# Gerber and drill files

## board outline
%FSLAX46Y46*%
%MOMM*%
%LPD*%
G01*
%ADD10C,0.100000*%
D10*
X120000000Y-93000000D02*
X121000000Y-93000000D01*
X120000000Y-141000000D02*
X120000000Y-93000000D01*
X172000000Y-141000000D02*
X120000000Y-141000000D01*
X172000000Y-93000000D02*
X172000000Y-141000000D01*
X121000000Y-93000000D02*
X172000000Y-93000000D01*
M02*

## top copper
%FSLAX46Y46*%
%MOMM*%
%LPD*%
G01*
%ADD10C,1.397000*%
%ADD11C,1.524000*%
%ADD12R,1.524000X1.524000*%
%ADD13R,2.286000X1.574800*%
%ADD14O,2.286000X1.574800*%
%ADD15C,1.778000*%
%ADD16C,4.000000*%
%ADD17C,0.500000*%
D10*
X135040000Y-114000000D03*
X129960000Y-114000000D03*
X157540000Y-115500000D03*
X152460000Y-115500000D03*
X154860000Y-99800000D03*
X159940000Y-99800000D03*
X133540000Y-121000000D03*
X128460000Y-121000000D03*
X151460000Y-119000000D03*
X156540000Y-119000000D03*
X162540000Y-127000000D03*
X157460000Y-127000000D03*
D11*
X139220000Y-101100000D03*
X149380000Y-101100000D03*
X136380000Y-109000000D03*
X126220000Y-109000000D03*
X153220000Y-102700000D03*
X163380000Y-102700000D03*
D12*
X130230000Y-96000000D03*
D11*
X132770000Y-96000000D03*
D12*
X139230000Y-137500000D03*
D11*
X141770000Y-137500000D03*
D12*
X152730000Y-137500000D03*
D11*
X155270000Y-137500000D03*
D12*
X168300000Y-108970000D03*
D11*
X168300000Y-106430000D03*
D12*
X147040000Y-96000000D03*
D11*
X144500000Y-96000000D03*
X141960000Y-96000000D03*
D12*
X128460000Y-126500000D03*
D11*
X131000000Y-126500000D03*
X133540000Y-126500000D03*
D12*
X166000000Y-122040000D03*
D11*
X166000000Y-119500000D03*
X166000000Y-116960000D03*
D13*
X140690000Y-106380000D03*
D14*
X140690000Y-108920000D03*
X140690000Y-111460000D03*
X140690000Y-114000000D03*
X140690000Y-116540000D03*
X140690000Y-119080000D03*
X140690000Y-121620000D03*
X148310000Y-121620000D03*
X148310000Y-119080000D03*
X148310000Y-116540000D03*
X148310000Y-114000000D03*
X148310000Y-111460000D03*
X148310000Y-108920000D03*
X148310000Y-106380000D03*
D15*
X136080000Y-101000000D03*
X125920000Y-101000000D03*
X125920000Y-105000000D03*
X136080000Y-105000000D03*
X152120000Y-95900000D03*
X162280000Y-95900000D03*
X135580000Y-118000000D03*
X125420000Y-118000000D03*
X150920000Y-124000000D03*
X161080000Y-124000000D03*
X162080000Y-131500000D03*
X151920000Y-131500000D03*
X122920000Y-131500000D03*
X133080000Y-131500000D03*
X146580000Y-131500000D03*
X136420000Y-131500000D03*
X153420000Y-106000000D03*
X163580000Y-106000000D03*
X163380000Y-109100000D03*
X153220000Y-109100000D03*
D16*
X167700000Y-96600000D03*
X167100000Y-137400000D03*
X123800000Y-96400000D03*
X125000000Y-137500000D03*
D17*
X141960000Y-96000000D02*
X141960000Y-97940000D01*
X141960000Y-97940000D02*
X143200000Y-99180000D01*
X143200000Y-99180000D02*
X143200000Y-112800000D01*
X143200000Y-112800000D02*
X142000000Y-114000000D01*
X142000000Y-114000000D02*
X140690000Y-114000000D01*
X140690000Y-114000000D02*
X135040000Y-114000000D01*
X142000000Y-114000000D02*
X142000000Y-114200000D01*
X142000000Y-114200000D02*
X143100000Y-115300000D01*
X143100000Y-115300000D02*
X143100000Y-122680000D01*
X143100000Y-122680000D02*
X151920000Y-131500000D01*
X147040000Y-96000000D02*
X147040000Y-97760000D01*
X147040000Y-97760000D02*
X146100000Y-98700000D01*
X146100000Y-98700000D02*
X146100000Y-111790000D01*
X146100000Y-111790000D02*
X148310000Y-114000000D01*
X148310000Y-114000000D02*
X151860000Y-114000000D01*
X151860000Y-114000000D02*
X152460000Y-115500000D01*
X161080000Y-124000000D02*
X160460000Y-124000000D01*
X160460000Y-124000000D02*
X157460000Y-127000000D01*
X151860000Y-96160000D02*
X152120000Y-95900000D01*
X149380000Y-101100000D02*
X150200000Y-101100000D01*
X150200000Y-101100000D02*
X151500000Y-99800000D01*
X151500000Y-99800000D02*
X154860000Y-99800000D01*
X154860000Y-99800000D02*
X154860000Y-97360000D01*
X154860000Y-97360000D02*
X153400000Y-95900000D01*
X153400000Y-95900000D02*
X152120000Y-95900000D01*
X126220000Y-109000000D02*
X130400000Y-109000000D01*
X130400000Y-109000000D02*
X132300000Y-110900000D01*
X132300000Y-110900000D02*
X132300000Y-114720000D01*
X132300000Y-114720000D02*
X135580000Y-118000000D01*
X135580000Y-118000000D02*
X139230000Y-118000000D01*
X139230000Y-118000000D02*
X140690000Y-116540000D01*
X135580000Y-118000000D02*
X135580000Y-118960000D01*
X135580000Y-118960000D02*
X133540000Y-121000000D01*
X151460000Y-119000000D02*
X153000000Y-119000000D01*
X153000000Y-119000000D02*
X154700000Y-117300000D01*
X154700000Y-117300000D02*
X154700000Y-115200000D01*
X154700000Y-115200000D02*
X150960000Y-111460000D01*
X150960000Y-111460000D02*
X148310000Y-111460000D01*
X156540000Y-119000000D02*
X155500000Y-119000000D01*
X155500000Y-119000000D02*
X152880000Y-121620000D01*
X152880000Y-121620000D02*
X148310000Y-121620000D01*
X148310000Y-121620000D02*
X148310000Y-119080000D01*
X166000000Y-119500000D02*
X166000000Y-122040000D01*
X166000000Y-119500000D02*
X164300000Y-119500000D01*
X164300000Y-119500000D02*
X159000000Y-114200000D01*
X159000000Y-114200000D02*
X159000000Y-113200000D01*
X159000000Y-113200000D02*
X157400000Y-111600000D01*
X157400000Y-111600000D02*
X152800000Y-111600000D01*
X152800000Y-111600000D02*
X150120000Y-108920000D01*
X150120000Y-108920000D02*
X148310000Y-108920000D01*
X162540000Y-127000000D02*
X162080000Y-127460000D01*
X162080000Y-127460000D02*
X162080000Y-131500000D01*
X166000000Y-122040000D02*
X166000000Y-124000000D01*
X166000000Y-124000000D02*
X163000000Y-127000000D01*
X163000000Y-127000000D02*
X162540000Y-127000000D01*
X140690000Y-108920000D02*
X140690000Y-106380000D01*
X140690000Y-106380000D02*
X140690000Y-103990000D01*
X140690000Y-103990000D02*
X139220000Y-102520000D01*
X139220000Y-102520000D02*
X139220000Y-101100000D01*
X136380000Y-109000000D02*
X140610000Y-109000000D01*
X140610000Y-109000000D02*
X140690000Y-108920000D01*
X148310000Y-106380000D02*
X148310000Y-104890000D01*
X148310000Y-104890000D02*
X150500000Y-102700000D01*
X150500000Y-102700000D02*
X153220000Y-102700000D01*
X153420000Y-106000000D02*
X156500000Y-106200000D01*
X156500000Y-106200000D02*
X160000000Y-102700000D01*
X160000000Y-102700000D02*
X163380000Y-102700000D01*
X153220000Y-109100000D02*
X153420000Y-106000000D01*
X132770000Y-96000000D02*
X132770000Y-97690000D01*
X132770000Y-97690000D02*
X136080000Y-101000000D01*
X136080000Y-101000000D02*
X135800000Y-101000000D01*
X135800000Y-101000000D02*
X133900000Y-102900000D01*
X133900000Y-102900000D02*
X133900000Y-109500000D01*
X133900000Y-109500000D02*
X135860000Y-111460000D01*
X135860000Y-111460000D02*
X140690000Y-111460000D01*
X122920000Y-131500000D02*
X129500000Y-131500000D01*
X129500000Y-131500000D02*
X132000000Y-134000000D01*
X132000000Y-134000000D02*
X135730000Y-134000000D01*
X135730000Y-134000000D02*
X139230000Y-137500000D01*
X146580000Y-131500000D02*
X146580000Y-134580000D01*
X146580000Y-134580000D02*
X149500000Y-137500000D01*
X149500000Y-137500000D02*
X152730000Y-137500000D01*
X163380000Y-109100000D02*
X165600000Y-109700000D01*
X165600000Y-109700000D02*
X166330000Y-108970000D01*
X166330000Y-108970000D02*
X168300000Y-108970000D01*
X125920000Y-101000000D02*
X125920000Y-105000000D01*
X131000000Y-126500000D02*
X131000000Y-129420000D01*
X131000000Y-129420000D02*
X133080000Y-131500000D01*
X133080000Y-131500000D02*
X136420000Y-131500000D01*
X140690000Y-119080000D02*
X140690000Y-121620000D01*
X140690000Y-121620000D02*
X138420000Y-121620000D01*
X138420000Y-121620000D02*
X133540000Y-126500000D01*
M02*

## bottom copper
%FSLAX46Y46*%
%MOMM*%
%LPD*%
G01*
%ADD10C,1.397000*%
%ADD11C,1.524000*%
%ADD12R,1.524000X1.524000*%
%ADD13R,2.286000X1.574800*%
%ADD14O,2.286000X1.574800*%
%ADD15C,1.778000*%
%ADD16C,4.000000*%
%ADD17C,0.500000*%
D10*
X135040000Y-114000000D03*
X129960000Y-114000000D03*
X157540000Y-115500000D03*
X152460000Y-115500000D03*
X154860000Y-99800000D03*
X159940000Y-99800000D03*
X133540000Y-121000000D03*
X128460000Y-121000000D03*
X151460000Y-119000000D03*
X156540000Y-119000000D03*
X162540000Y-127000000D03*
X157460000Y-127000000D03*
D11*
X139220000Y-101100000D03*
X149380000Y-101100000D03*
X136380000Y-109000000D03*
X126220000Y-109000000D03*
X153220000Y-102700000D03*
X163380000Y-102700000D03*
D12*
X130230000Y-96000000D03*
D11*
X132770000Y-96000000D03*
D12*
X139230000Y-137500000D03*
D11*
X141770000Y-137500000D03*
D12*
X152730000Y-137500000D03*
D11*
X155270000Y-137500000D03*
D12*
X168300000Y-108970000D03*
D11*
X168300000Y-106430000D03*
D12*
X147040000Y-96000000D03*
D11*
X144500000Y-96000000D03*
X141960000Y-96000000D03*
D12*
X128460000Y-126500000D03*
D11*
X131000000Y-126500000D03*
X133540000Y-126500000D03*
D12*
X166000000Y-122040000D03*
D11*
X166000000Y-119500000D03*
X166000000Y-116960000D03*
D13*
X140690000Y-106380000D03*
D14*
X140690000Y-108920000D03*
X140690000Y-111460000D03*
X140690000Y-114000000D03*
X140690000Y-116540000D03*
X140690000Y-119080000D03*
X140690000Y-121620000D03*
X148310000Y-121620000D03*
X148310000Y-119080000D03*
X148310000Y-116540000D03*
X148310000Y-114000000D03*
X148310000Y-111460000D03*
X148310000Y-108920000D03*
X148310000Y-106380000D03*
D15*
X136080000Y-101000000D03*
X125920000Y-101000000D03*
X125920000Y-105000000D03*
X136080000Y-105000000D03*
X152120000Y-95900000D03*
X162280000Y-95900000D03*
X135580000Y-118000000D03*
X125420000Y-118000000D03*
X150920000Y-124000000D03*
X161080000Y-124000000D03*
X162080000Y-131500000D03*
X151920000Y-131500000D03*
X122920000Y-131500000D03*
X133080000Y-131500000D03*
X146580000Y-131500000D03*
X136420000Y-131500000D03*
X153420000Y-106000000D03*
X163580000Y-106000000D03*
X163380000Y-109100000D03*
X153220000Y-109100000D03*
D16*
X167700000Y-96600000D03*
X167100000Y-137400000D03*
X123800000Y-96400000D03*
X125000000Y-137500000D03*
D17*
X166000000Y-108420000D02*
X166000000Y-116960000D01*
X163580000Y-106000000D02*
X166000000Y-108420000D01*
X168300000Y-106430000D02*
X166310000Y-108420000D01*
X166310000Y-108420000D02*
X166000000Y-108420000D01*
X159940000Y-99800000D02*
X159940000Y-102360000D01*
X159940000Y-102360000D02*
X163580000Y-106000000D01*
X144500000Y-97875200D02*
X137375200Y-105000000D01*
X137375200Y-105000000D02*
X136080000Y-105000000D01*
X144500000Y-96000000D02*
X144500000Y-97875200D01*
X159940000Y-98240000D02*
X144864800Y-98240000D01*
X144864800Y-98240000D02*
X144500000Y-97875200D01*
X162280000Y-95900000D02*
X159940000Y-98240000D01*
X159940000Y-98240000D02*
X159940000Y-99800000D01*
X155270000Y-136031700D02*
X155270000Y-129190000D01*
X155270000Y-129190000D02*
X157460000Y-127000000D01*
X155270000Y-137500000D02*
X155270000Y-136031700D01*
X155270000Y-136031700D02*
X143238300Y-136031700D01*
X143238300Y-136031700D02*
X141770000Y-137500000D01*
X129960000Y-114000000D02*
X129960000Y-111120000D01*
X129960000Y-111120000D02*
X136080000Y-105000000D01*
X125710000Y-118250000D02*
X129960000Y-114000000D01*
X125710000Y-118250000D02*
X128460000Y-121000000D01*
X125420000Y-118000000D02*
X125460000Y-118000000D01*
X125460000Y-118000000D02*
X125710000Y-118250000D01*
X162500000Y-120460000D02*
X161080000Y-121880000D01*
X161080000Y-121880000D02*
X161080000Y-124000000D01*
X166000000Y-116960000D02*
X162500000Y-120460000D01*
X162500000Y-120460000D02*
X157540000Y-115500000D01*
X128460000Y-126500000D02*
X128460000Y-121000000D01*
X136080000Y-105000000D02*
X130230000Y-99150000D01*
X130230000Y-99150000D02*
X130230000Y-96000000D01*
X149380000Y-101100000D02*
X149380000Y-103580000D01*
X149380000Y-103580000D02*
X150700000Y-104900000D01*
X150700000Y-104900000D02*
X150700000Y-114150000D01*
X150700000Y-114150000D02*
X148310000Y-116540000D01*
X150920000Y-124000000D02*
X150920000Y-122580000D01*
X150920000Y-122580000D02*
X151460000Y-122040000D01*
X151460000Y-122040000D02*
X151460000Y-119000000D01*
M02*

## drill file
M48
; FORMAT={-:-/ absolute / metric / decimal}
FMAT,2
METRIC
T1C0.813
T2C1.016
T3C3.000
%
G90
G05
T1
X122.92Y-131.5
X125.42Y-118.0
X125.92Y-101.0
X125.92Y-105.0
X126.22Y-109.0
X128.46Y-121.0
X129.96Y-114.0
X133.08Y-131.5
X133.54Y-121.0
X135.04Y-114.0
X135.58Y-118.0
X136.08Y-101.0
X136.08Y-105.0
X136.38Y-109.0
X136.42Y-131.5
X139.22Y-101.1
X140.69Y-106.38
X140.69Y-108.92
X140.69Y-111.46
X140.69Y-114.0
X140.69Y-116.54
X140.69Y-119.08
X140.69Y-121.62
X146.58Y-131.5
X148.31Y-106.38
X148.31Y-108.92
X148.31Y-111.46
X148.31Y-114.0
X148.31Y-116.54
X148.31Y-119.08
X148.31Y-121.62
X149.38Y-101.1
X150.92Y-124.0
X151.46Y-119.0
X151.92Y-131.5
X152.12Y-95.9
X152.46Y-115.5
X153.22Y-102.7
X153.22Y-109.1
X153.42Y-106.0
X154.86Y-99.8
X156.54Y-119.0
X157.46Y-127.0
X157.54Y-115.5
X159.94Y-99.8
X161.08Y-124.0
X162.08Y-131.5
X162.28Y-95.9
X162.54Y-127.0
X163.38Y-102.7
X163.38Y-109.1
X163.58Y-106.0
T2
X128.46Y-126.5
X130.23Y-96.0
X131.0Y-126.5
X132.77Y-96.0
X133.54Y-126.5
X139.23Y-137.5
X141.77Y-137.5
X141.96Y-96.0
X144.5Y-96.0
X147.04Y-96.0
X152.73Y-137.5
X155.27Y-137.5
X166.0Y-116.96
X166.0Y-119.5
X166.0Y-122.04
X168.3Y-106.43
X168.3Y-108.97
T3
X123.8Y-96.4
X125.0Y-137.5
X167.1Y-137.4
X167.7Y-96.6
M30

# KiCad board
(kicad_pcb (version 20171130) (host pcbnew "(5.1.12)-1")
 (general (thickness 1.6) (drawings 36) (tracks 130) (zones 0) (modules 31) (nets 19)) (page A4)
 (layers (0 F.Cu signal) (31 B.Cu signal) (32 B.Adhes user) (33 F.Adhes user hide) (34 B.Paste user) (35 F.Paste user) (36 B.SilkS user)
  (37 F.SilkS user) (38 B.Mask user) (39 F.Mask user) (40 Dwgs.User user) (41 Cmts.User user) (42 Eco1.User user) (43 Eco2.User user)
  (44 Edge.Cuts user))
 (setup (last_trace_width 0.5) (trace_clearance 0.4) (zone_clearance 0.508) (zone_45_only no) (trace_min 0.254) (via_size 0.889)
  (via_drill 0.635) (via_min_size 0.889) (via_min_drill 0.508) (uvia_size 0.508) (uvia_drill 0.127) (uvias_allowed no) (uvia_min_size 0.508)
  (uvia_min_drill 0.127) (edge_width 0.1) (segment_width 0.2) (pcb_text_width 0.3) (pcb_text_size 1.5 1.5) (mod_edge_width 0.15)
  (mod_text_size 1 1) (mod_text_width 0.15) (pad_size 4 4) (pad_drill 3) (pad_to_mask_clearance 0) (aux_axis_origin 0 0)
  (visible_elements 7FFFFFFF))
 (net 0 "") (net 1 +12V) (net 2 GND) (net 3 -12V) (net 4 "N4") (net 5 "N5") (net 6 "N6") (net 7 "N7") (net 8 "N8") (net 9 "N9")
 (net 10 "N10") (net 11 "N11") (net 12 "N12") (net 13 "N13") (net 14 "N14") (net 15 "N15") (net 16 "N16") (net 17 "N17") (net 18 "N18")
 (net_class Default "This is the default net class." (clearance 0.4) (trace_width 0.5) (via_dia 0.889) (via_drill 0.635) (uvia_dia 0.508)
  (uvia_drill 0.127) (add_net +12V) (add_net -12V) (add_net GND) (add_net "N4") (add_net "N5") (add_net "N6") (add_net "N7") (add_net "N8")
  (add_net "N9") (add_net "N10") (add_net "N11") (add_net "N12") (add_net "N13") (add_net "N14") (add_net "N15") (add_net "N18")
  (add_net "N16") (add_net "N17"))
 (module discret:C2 (layer F.Cu) (at 132.5 114 180)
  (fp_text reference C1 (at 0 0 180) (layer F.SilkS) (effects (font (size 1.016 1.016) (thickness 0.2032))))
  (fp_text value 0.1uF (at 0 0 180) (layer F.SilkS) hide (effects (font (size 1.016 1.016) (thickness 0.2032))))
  (pad 1 thru_hole circle (at -2.54 0 180) (size 1.397 1.397) (drill 0.8128) (layers *.Cu *.Mask F.SilkS) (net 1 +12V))
  (pad 2 thru_hole circle (at 2.54 0 180) (size 1.397 1.397) (drill 0.8128) (layers *.Cu *.Mask F.SilkS) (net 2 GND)))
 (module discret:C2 (layer F.Cu) (at 155 115.5 180)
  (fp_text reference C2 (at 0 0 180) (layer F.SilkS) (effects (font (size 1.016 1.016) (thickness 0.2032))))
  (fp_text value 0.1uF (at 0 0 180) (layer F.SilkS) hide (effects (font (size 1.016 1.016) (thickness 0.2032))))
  (pad 1 thru_hole circle (at -2.54 0 180) (size 1.397 1.397) (drill 0.8128) (layers *.Cu *.Mask F.SilkS) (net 2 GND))
  (pad 2 thru_hole circle (at 2.54 0 180) (size 1.397 1.397) (drill 0.8128) (layers *.Cu *.Mask F.SilkS) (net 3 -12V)))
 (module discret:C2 (layer F.Cu) (at 157.4 99.8)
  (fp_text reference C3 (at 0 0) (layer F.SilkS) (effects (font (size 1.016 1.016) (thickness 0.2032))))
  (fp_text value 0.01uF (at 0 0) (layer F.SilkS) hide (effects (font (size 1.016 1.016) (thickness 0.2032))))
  (pad 1 thru_hole circle (at -2.54 0) (size 1.397 1.397) (drill 0.8128) (layers *.Cu *.Mask F.SilkS) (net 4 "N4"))
  (pad 2 thru_hole circle (at 2.54 0) (size 1.397 1.397) (drill 0.8128) (layers *.Cu *.Mask F.SilkS) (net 2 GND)))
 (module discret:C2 (layer F.Cu) (at 131 121 180)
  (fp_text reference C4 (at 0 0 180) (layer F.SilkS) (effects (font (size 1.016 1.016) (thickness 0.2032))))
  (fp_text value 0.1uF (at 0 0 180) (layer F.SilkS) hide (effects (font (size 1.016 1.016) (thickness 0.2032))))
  (pad 1 thru_hole circle (at -2.54 0 180) (size 1.397 1.397) (drill 0.8128) (layers *.Cu *.Mask F.SilkS) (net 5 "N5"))
  (pad 2 thru_hole circle (at 2.54 0 180) (size 1.397 1.397) (drill 0.8128) (layers *.Cu *.Mask F.SilkS) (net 2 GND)))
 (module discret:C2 (layer F.Cu) (at 154 119)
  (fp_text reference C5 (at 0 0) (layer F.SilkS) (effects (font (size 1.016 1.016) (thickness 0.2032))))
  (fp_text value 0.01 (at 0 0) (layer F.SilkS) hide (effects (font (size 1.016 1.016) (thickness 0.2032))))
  (pad 1 thru_hole circle (at -2.54 0) (size 1.397 1.397) (drill 0.8128) (layers *.Cu *.Mask F.SilkS) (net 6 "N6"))
  (pad 2 thru_hole circle (at 2.54 0) (size 1.397 1.397) (drill 0.8128) (layers *.Cu *.Mask F.SilkS) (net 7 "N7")))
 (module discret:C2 (layer F.Cu) (at 160 127 180)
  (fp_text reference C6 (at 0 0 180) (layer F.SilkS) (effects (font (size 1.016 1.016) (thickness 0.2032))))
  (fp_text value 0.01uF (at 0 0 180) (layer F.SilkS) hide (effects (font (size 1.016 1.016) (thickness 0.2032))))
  (pad 1 thru_hole circle (at -2.54 0 180) (size 1.397 1.397) (drill 0.8128) (layers *.Cu *.Mask F.SilkS) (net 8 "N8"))
  (pad 2 thru_hole circle (at 2.54 0 180) (size 1.397 1.397) (drill 0.8128) (layers *.Cu *.Mask F.SilkS) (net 2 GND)))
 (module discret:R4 (layer F.Cu) (at 144.3 101.1) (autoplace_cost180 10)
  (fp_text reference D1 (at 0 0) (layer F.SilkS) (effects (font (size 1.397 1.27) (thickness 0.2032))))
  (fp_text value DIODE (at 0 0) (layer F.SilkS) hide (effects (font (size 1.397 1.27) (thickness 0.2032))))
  (pad 1 thru_hole circle (at -5.08 0) (size 1.524 1.524) (drill 0.8128) (layers *.Cu *.Mask F.SilkS) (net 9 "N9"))
  (pad 2 thru_hole circle (at 5.08 0) (size 1.524 1.524) (drill 0.8128) (layers *.Cu *.Mask F.SilkS) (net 4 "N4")))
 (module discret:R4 (layer F.Cu) (at 131.3 109 180) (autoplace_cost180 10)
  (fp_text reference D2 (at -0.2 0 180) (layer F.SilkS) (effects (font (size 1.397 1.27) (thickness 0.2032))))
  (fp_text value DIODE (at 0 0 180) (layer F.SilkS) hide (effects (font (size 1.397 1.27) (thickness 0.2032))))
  (pad 1 thru_hole circle (at -5.08 0 180) (size 1.524 1.524) (drill 0.8128) (layers *.Cu *.Mask F.SilkS) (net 9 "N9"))
  (pad 2 thru_hole circle (at 5.08 0 180) (size 1.524 1.524) (drill 0.8128) (layers *.Cu *.Mask F.SilkS) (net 5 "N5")))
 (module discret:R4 (layer F.Cu) (at 158.3 102.7) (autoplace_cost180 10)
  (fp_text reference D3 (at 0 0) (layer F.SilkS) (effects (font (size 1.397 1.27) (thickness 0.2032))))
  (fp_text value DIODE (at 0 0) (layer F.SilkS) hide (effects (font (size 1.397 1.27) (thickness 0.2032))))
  (pad 1 thru_hole circle (at -5.08 0) (size 1.524 1.524) (drill 0.8128) (layers *.Cu *.Mask F.SilkS) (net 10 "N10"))
  (pad 2 thru_hole circle (at 5.08 0) (size 1.524 1.524) (drill 0.8128) (layers *.Cu *.Mask F.SilkS) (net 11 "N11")))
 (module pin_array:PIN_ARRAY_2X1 (layer F.Cu) (at 131.5 96)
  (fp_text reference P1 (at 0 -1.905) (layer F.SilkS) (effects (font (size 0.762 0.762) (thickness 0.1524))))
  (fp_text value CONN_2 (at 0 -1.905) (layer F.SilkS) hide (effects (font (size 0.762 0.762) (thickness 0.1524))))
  (pad 1 thru_hole rect (at -1.27 0) (size 1.524 1.524) (drill 1.016) (layers *.Cu *.Mask F.SilkS) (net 2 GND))
  (pad 2 thru_hole circle (at 1.27 0) (size 1.524 1.524) (drill 1.016) (layers *.Cu *.Mask F.SilkS) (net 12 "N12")))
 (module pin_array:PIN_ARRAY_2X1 (layer F.Cu) (at 140.5 137.5)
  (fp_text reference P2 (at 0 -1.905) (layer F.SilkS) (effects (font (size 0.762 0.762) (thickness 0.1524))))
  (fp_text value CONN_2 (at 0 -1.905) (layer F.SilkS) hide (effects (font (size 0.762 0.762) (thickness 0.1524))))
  (pad 1 thru_hole rect (at -1.27 0) (size 1.524 1.524) (drill 1.016) (layers *.Cu *.Mask F.SilkS) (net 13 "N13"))
  (pad 2 thru_hole circle (at 1.27 0) (size 1.524 1.524) (drill 1.016) (layers *.Cu *.Mask F.SilkS) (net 2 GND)))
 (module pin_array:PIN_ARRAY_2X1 (layer F.Cu) (at 154 137.5)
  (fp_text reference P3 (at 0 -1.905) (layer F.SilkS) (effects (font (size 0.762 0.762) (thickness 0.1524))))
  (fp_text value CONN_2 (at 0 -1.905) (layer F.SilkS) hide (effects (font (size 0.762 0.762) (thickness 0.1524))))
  (pad 1 thru_hole rect (at -1.27 0) (size 1.524 1.524) (drill 1.016) (layers *.Cu *.Mask F.SilkS) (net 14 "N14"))
  (pad 2 thru_hole circle (at 1.27 0) (size 1.524 1.524) (drill 1.016) (layers *.Cu *.Mask F.SilkS) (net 2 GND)))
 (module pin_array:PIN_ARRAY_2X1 (layer F.Cu) (at 168.3 107.7 90)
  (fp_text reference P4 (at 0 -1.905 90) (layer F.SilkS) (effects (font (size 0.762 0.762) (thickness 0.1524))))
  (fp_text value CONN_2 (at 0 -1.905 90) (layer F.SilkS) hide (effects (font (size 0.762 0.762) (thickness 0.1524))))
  (pad 1 thru_hole rect (at -1.27 0 90) (size 1.524 1.524) (drill 1.016) (layers *.Cu *.Mask F.SilkS) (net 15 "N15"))
  (pad 2 thru_hole circle (at 1.27 0 90) (size 1.524 1.524) (drill 1.016) (layers *.Cu *.Mask F.SilkS) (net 2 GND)))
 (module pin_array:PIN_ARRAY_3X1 (layer F.Cu) (at 144.5 96 180)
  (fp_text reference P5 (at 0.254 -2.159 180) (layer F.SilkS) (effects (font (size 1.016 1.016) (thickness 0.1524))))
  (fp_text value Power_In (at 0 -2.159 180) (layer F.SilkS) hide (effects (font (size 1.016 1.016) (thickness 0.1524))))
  (pad 1 thru_hole rect (at -2.54 0 180) (size 1.524 1.524) (drill 1.016) (layers *.Cu *.Mask F.SilkS) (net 3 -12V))
  (pad 2 thru_hole circle (at 0 0 180) (size 1.524 1.524) (drill 1.016) (layers *.Cu *.Mask F.SilkS) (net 2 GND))
  (pad 3 thru_hole circle (at 2.54 0 180) (size 1.524 1.524) (drill 1.016) (layers *.Cu *.Mask F.SilkS) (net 1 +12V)))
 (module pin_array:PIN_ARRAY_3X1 (layer F.Cu) (at 131 126.5)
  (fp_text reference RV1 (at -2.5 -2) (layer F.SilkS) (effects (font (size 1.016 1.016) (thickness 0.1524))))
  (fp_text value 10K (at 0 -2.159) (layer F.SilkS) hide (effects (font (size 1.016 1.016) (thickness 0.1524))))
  (pad 1 thru_hole rect (at -2.54 0) (size 1.524 1.524) (drill 1.016) (layers *.Cu *.Mask F.SilkS) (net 2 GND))
  (pad 2 thru_hole circle (at 0 0) (size 1.524 1.524) (drill 1.016) (layers *.Cu *.Mask F.SilkS) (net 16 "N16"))
  (pad 3 thru_hole circle (at 2.54 0) (size 1.524 1.524) (drill 1.016) (layers *.Cu *.Mask F.SilkS) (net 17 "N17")))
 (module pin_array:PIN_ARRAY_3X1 (layer F.Cu) (at 166 119.5 90)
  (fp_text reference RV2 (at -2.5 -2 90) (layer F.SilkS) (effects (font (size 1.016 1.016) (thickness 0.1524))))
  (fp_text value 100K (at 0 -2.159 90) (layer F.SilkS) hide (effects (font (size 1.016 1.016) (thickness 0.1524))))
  (pad 1 thru_hole rect (at -2.54 0 90) (size 1.524 1.524) (drill 1.016) (layers *.Cu *.Mask F.SilkS) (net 8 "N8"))
  (pad 2 thru_hole circle (at 0 0 90) (size 1.524 1.524) (drill 1.016) (layers *.Cu *.Mask F.SilkS) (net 8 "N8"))
  (pad 3 thru_hole circle (at 2.54 0 90) (size 1.524 1.524) (drill 1.016) (layers *.Cu *.Mask F.SilkS) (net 2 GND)))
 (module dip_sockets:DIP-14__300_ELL (layer F.Cu) (at 144.5 114 270)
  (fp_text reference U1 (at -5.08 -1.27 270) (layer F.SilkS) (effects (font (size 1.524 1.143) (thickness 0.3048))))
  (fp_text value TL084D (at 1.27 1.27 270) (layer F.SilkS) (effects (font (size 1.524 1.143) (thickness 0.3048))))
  (pad 1 thru_hole rect (at -7.62 3.81 270) (size 1.5748 2.286) (drill 0.8128) (layers *.Cu *.Mask F.SilkS) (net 9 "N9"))
  (pad 2 thru_hole oval (at -5.08 3.81 270) (size 1.5748 2.286) (drill 0.8128) (layers *.Cu *.Mask F.SilkS) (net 9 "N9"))
  (pad 3 thru_hole oval (at -2.54 3.81 270) (size 1.5748 2.286) (drill 0.8128) (layers *.Cu *.Mask F.SilkS) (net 12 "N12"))
  (pad 4 thru_hole oval (at 0 3.81 270) (size 1.5748 2.286) (drill 0.8128) (layers *.Cu *.Mask F.SilkS) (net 1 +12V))
  (pad 5 thru_hole oval (at 2.54 3.81 270) (size 1.5748 2.286) (drill 0.8128) (layers *.Cu *.Mask F.SilkS) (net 5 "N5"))
  (pad 6 thru_hole oval (at 5.08 3.81 270) (size 1.5748 2.286) (drill 0.8128) (layers *.Cu *.Mask F.SilkS) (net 17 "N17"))
  (pad 7 thru_hole oval (at 7.62 3.81 270) (size 1.5748 2.286) (drill 0.8128) (layers *.Cu *.Mask F.SilkS) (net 17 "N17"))
  (pad 8 thru_hole oval (at 7.62 -3.81 270) (size 1.5748 2.286) (drill 0.8128) (layers *.Cu *.Mask F.SilkS) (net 7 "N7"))
  (pad 9 thru_hole oval (at 5.08 -3.81 270) (size 1.5748 2.286) (drill 0.8128) (layers *.Cu *.Mask F.SilkS) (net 7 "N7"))
  (pad 10 thru_hole oval (at 2.54 -3.81 270) (size 1.5748 2.286) (drill 0.8128) (layers *.Cu *.Mask F.SilkS) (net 4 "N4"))
  (pad 11 thru_hole oval (at 0 -3.81 270) (size 1.5748 2.286) (drill 0.8128) (layers *.Cu *.Mask F.SilkS) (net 3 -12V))
  (pad 12 thru_hole oval (at -2.54 -3.81 270) (size 1.5748 2.286) (drill 0.8128) (layers *.Cu *.Mask F.SilkS) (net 6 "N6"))
  (pad 13 thru_hole oval (at -5.08 -3.81 270) (size 1.5748 2.286) (drill 0.8128) (layers *.Cu *.Mask F.SilkS) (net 8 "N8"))
  (pad 14 thru_hole oval (at -7.62 -3.81 270) (size 1.5748 2.286) (drill 0.8128) (layers *.Cu *.Mask F.SilkS) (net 10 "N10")))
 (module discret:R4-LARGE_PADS (layer F.Cu) (at 131 101 180) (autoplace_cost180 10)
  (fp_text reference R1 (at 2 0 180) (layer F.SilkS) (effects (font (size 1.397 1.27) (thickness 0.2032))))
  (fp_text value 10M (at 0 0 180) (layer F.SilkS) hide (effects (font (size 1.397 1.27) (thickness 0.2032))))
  (pad 1 thru_hole circle (at -5.08 0 180) (size 1.778 1.778) (drill 0.8128) (layers *.Cu *.Mask F.SilkS) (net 12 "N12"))
  (pad 2 thru_hole circle (at 5.08 0 180) (size 1.778 1.778) (drill 0.8128) (layers *.Cu *.Mask F.SilkS) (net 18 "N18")))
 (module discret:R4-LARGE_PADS (layer F.Cu) (at 131 105) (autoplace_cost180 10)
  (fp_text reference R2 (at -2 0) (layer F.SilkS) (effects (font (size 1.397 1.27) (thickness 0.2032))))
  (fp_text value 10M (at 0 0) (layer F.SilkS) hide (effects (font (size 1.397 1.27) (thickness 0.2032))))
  (pad 1 thru_hole circle (at -5.08 0) (size 1.778 1.778) (drill 0.8128) (layers *.Cu *.Mask F.SilkS) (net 18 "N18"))
  (pad 2 thru_hole circle (at 5.08 0) (size 1.778 1.778) (drill 0.8128) (layers *.Cu *.Mask F.SilkS) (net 2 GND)))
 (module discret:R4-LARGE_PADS (layer F.Cu) (at 157.2 95.9) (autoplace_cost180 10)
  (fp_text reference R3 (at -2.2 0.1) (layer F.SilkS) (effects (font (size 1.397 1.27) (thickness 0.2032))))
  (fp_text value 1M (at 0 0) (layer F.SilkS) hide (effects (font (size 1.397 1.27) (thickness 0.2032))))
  (pad 1 thru_hole circle (at -5.08 0) (size 1.778 1.778) (drill 0.8128) (layers *.Cu *.Mask F.SilkS) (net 4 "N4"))
  (pad 2 thru_hole circle (at 5.08 0) (size 1.778 1.778) (drill 0.8128) (layers *.Cu *.Mask F.SilkS) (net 2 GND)))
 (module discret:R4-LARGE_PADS (layer F.Cu) (at 130.5 118 180) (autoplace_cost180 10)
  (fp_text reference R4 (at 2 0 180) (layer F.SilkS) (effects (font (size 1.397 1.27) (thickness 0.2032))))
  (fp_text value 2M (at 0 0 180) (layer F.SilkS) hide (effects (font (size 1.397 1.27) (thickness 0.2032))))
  (pad 1 thru_hole circle (at -5.08 0 180) (size 1.778 1.778) (drill 0.8128) (layers *.Cu *.Mask F.SilkS) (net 5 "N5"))
  (pad 2 thru_hole circle (at 5.08 0 180) (size 1.778 1.778) (drill 0.8128) (layers *.Cu *.Mask F.SilkS) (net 2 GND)))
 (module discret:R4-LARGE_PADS (layer F.Cu) (at 156 124) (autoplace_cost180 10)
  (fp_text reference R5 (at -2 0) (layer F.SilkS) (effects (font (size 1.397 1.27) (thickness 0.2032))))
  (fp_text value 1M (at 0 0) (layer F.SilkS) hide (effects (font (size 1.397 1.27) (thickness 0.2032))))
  (pad 1 thru_hole circle (at -5.08 0) (size 1.778 1.778) (drill 0.8128) (layers *.Cu *.Mask F.SilkS) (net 6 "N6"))
  (pad 2 thru_hole circle (at 5.08 0) (size 1.778 1.778) (drill 0.8128) (layers *.Cu *.Mask F.SilkS) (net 2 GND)))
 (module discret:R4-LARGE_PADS (layer F.Cu) (at 157 131.5 180) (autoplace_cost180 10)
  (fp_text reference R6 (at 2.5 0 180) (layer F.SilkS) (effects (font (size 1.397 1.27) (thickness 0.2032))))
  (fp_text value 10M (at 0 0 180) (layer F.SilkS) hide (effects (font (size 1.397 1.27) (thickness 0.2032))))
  (pad 1 thru_hole circle (at -5.08 0 180) (size 1.778 1.778) (drill 0.8128) (layers *.Cu *.Mask F.SilkS) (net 8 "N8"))
  (pad 2 thru_hole circle (at 5.08 0 180) (size 1.778 1.778) (drill 0.8128) (layers *.Cu *.Mask F.SilkS) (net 1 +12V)))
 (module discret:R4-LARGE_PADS (layer F.Cu) (at 128 131.5) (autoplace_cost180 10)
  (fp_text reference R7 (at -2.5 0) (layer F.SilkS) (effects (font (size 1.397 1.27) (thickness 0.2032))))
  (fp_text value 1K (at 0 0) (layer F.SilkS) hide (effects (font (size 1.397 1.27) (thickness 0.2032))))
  (pad 1 thru_hole circle (at -5.08 0) (size 1.778 1.778) (drill 0.8128) (layers *.Cu *.Mask F.SilkS) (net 13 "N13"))
  (pad 2 thru_hole circle (at 5.08 0) (size 1.778 1.778) (drill 0.8128) (layers *.Cu *.Mask F.SilkS) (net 16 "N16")))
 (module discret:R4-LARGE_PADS (layer F.Cu) (at 141.5 131.5 180) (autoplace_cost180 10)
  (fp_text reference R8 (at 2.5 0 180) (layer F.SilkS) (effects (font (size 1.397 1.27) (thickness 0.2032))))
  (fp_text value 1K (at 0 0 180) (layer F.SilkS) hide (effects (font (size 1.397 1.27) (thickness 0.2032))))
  (pad 1 thru_hole circle (at -5.08 0 180) (size 1.778 1.778) (drill 0.8128) (layers *.Cu *.Mask F.SilkS) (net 14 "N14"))
  (pad 2 thru_hole circle (at 5.08 0 180) (size 1.778 1.778) (drill 0.8128) (layers *.Cu *.Mask F.SilkS) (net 16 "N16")))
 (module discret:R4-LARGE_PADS (layer F.Cu) (at 158.5 106) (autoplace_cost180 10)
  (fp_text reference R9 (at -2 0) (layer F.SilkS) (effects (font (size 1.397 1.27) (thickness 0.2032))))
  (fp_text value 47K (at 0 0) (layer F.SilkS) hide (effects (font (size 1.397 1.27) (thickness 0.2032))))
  (pad 1 thru_hole circle (at -5.08 0) (size 1.778 1.778) (drill 0.8128) (layers *.Cu *.Mask F.SilkS) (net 11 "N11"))
  (pad 2 thru_hole circle (at 5.08 0) (size 1.778 1.778) (drill 0.8128) (layers *.Cu *.Mask F.SilkS) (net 2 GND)))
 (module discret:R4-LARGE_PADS (layer F.Cu) (at 158.3 109.1 180) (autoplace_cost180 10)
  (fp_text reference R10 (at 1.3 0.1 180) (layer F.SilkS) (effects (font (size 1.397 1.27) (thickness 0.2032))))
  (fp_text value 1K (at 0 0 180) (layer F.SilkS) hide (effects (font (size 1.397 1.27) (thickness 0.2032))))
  (pad 1 thru_hole circle (at -5.08 0 180) (size 1.778 1.778) (drill 0.8128) (layers *.Cu *.Mask F.SilkS) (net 15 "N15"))
  (pad 2 thru_hole circle (at 5.08 0 180) (size 1.778 1.778) (drill 0.8128) (layers *.Cu *.Mask F.SilkS) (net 11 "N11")))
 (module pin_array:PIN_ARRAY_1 (layer F.Cu) (at 167.7 96.6 90)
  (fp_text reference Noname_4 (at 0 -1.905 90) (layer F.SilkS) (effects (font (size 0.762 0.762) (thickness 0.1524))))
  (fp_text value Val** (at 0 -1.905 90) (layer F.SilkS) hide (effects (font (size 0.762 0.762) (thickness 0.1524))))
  (pad 1 thru_hole circle (at 0 0 90) (size 4 4) (drill 3) (layers *.Cu *.Mask F.SilkS)))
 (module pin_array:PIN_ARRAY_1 (layer F.Cu) (at 167.1 137.4)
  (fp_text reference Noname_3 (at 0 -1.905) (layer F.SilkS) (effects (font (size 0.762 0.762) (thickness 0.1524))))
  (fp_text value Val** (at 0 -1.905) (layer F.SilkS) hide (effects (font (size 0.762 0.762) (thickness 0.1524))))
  (pad 1 thru_hole circle (at 0 0) (size 4 4) (drill 3) (layers *.Cu *.Mask F.SilkS)))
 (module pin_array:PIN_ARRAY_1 (layer F.Cu) (at 123.8 96.4)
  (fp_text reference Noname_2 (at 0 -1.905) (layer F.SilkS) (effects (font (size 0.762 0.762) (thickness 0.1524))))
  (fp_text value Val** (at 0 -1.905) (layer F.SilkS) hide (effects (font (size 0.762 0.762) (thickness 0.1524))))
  (pad 1 thru_hole circle (at 0 0) (size 4 4) (drill 3) (layers *.Cu *.Mask F.SilkS)))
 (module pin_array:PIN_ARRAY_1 (layer F.Cu) (at 125 137.5)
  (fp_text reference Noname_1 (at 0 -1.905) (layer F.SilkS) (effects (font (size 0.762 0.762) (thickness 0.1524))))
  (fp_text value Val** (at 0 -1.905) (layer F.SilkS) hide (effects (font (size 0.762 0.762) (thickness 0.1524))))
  (pad 1 thru_hole circle (at 0 0) (size 4 4) (drill 3) (layers *.Cu *.Mask F.SilkS)))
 (gr_line (start 120 93) (end 121 93) (angle 90) (layer Edge.Cuts) (width 0.1))
 (gr_line (start 120 141) (end 120 93) (angle 90) (layer Edge.Cuts) (width 0.1))
 (gr_line (start 172 141) (end 120 141) (angle 90) (layer Edge.Cuts) (width 0.1))
 (gr_line (start 172 93) (end 172 141) (angle 90) (layer Edge.Cuts) (width 0.1))
 (gr_line (start 121 93) (end 172 93) (angle 90) (layer Edge.Cuts) (width 0.1))
 (segment (start 141.96 96) (end 141.96 97.94) (width 0.5) (layer F.Cu) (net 1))
 (segment (start 141.96 97.94) (end 143.2 99.18) (width 0.5) (layer F.Cu) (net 1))
 (segment (start 143.2 99.18) (end 143.2 112.8) (width 0.5) (layer F.Cu) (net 1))
 (segment (start 143.2 112.8) (end 142 114) (width 0.5) (layer F.Cu) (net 1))
 (segment (start 142 114) (end 140.69 114) (width 0.5) (layer F.Cu) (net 1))
 (segment (start 140.69 114) (end 135.04 114) (width 0.5) (layer F.Cu) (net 1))
 (segment (start 142 114) (end 142 114.2) (width 0.5) (layer F.Cu) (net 1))
 (segment (start 142 114.2) (end 143.1 115.3) (width 0.5) (layer F.Cu) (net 1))
 (segment (start 143.1 115.3) (end 143.1 122.68) (width 0.5) (layer F.Cu) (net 1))
 (segment (start 143.1 122.68) (end 151.92 131.5) (width 0.5) (layer F.Cu) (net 1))
 (segment (start 147.04 96) (end 147.04 97.76) (width 0.5) (layer F.Cu) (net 3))
 (segment (start 147.04 97.76) (end 146.1 98.7) (width 0.5) (layer F.Cu) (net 3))
 (segment (start 146.1 98.7) (end 146.1 111.79) (width 0.5) (layer F.Cu) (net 3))
 (segment (start 146.1 111.79) (end 148.31 114) (width 0.5) (layer F.Cu) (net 3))
 (segment (start 148.31 114) (end 151.86 114) (width 0.5) (layer F.Cu) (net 3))
 (segment (start 151.86 114) (end 152.46 115.5) (width 0.5) (layer F.Cu) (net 3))
 (segment (start 166 108.42) (end 166 116.96) (width 0.5) (layer B.Cu) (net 2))
 (segment (start 163.58 106) (end 166 108.42) (width 0.5) (layer B.Cu) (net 2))
 (segment (start 168.3 106.43) (end 166.31 108.42) (width 0.5) (layer B.Cu) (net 2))
 (segment (start 166.31 108.42) (end 166 108.42) (width 0.5) (layer B.Cu) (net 2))
 (segment (start 159.94 99.8) (end 159.94 102.36) (width 0.5) (layer B.Cu) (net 2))
 (segment (start 159.94 102.36) (end 163.58 106) (width 0.5) (layer B.Cu) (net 2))
 (segment (start 144.5 97.8752) (end 137.3752 105) (width 0.5) (layer B.Cu) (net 2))
 (segment (start 137.3752 105) (end 136.08 105) (width 0.5) (layer B.Cu) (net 2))
 (segment (start 144.5 96) (end 144.5 97.8752) (width 0.5) (layer B.Cu) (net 2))
 (segment (start 159.94 98.24) (end 144.8648 98.24) (width 0.5) (layer B.Cu) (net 2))
 (segment (start 144.8648 98.24) (end 144.5 97.8752) (width 0.5) (layer B.Cu) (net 2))
 (segment (start 162.28 95.9) (end 159.94 98.24) (width 0.5) (layer B.Cu) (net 2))
 (segment (start 159.94 98.24) (end 159.94 99.8) (width 0.5) (layer B.Cu) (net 2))
 (segment (start 155.27 136.0317) (end 155.27 129.19) (width 0.5) (layer B.Cu) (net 2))
 (segment (start 155.27 129.19) (end 157.46 127) (width 0.5) (layer B.Cu) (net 2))
 (segment (start 155.27 137.5) (end 155.27 136.0317) (width 0.5) (layer B.Cu) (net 2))
 (segment (start 155.27 136.0317) (end 143.2383 136.0317) (width 0.5) (layer B.Cu) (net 2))
 (segment (start 143.2383 136.0317) (end 141.77 137.5) (width 0.5) (layer B.Cu) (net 2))
 (segment (start 129.96 114) (end 129.96 111.12) (width 0.5) (layer B.Cu) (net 2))
 (segment (start 129.96 111.12) (end 136.08 105) (width 0.5) (layer B.Cu) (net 2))
 (segment (start 125.71 118.25) (end 129.96 114) (width 0.5) (layer B.Cu) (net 2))
 (segment (start 125.71 118.25) (end 128.46 121) (width 0.5) (layer B.Cu) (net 2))
 (segment (start 125.42 118) (end 125.46 118) (width 0.5) (layer B.Cu) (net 2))
 (segment (start 125.46 118) (end 125.71 118.25) (width 0.5) (layer B.Cu) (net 2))
 (segment (start 162.5 120.46) (end 161.08 121.88) (width 0.5) (layer B.Cu) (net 2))
 (segment (start 161.08 121.88) (end 161.08 124) (width 0.5) (layer B.Cu) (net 2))
 (segment (start 166 116.96) (end 162.5 120.46) (width 0.5) (layer B.Cu) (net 2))
 (segment (start 162.5 120.46) (end 157.54 115.5) (width 0.5) (layer B.Cu) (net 2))
 (segment (start 128.46 126.5) (end 128.46 121) (width 0.5) (layer B.Cu) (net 2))
 (segment (start 136.08 105) (end 130.23 99.15) (width 0.5) (layer B.Cu) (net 2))
 (segment (start 130.23 99.15) (end 130.23 96) (width 0.5) (layer B.Cu) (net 2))
 (segment (start 161.08 124) (end 160.46 124) (width 0.5) (layer F.Cu) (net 2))
 (segment (start 160.46 124) (end 157.46 127) (width 0.5) (layer F.Cu) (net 2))
 (segment (start 151.86 96.16) (end 152.12 95.9) (width 0.5) (layer F.Cu) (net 4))
 (segment (start 149.38 101.1) (end 149.38 103.58) (width 0.5) (layer B.Cu) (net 4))
 (segment (start 149.38 103.58) (end 150.7 104.9) (width 0.5) (layer B.Cu) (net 4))
 (segment (start 150.7 104.9) (end 150.7 114.15) (width 0.5) (layer B.Cu) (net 4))
 (segment (start 150.7 114.15) (end 148.31 116.54) (width 0.5) (layer B.Cu) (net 4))
 (segment (start 149.38 101.1) (end 150.2 101.1) (width 0.5) (layer F.Cu) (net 4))
 (segment (start 150.2 101.1) (end 151.5 99.8) (width 0.5) (layer F.Cu) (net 4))
 (segment (start 151.5 99.8) (end 154.86 99.8) (width 0.5) (layer F.Cu) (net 4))
 (segment (start 154.86 99.8) (end 154.86 97.36) (width 0.5) (layer F.Cu) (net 4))
 (segment (start 154.86 97.36) (end 153.4 95.9) (width 0.5) (layer F.Cu) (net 4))
 (segment (start 153.4 95.9) (end 152.12 95.9) (width 0.5) (layer F.Cu) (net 4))
 (segment (start 126.22 109) (end 130.4 109) (width 0.5) (layer F.Cu) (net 5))
 (segment (start 130.4 109) (end 132.3 110.9) (width 0.5) (layer F.Cu) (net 5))
 (segment (start 132.3 110.9) (end 132.3 114.72) (width 0.5) (layer F.Cu) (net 5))
 (segment (start 132.3 114.72) (end 135.58 118) (width 0.5) (layer F.Cu) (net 5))
 (segment (start 135.58 118) (end 139.23 118) (width 0.5) (layer F.Cu) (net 5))
 (segment (start 139.23 118) (end 140.69 116.54) (width 0.5) (layer F.Cu) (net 5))
 (segment (start 135.58 118) (end 135.58 118.96) (width 0.5) (layer F.Cu) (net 5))
 (segment (start 135.58 118.96) (end 133.54 121) (width 0.5) (layer F.Cu) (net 5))
 (segment (start 151.46 119) (end 153 119) (width 0.5) (layer F.Cu) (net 6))
 (segment (start 153 119) (end 154.7 117.3) (width 0.5) (layer F.Cu) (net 6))
 (segment (start 154.7 117.3) (end 154.7 115.2) (width 0.5) (layer F.Cu) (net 6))
 (segment (start 154.7 115.2) (end 150.96 111.46) (width 0.5) (layer F.Cu) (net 6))
 (segment (start 150.96 111.46) (end 148.31 111.46) (width 0.5) (layer F.Cu) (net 6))
 (segment (start 150.92 124) (end 150.92 122.58) (width 0.5) (layer B.Cu) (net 6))
 (segment (start 150.92 122.58) (end 151.46 122.04) (width 0.5) (layer B.Cu) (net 6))
 (segment (start 151.46 122.04) (end 151.46 119) (width 0.5) (layer B.Cu) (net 6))
 (segment (start 156.54 119) (end 155.5 119) (width 0.5) (layer F.Cu) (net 7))
 (segment (start 155.5 119) (end 152.88 121.62) (width 0.5) (layer F.Cu) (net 7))
 (segment (start 152.88 121.62) (end 148.31 121.62) (width 0.5) (layer F.Cu) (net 7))
 (segment (start 148.31 121.62) (end 148.31 119.08) (width 0.5) (layer F.Cu) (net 7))
 (segment (start 166 119.5) (end 166 122.04) (width 0.5) (layer F.Cu) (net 8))
 (segment (start 166 119.5) (end 164.3 119.5) (width 0.5) (layer F.Cu) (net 8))
 (segment (start 164.3 119.5) (end 159 114.2) (width 0.5) (layer F.Cu) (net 8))
 (segment (start 159 114.2) (end 159 113.2) (width 0.5) (layer F.Cu) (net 8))
 (segment (start 159 113.2) (end 157.4 111.6) (width 0.5) (layer F.Cu) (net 8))
 (segment (start 157.4 111.6) (end 152.8 111.6) (width 0.5) (layer F.Cu) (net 8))
 (segment (start 152.8 111.6) (end 150.12 108.92) (width 0.5) (layer F.Cu) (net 8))
 (segment (start 150.12 108.92) (end 148.31 108.92) (width 0.5) (layer F.Cu) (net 8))
 (segment (start 162.54 127) (end 162.08 127.46) (width 0.5) (layer F.Cu) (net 8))
 (segment (start 162.08 127.46) (end 162.08 131.5) (width 0.5) (layer F.Cu) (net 8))
 (segment (start 166 122.04) (end 166 124) (width 0.5) (layer F.Cu) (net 8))
 (segment (start 166 124) (end 163 127) (width 0.5) (layer F.Cu) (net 8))
 (segment (start 163 127) (end 162.54 127) (width 0.5) (layer F.Cu) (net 8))
 (segment (start 140.69 108.92) (end 140.69 106.38) (width 0.5) (layer F.Cu) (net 9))
 (segment (start 140.69 106.38) (end 140.69 103.99) (width 0.5) (layer F.Cu) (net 9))
 (segment (start 140.69 103.99) (end 139.22 102.52) (width 0.5) (layer F.Cu) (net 9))
 (segment (start 139.22 102.52) (end 139.22 101.1) (width 0.5) (layer F.Cu) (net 9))
 (segment (start 136.38 109) (end 140.61 109) (width 0.5) (layer F.Cu) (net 9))
 (segment (start 140.61 109) (end 140.69 108.92) (width 0.5) (layer F.Cu) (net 9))
 (segment (start 148.31 106.38) (end 148.31 104.89) (width 0.5) (layer F.Cu) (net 10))
 (segment (start 148.31 104.89) (end 150.5 102.7) (width 0.5) (layer F.Cu) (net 10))
 (segment (start 150.5 102.7) (end 153.22 102.7) (width 0.5) (layer F.Cu) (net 10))
 (segment (start 153.42 106) (end 156.5 106.2) (width 0.5) (layer F.Cu) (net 11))
 (segment (start 156.5 106.2) (end 160 102.7) (width 0.5) (layer F.Cu) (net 11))
 (segment (start 160 102.7) (end 163.38 102.7) (width 0.5) (layer F.Cu) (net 11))
 (segment (start 153.22 109.1) (end 153.42 106) (width 0.5) (layer F.Cu) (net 11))
 (segment (start 132.77 96) (end 132.77 97.69) (width 0.5) (layer F.Cu) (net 12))
 (segment (start 132.77 97.69) (end 136.08 101) (width 0.5) (layer F.Cu) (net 12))
 (segment (start 136.08 101) (end 135.8 101) (width 0.5) (layer F.Cu) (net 12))
 (segment (start 135.8 101) (end 133.9 102.9) (width 0.5) (layer F.Cu) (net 12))
 (segment (start 133.9 102.9) (end 133.9 109.5) (width 0.5) (layer F.Cu) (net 12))
 (segment (start 133.9 109.5) (end 135.86 111.46) (width 0.5) (layer F.Cu) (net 12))
 (segment (start 135.86 111.46) (end 140.69 111.46) (width 0.5) (layer F.Cu) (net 12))
 (segment (start 122.92 131.5) (end 129.5 131.5) (width 0.5) (layer F.Cu) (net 13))
 (segment (start 129.5 131.5) (end 132 134) (width 0.5) (layer F.Cu) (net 13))
 (segment (start 132 134) (end 135.73 134) (width 0.5) (layer F.Cu) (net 13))
 (segment (start 135.73 134) (end 139.23 137.5) (width 0.5) (layer F.Cu) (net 13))
 (segment (start 146.58 131.5) (end 146.58 134.58) (width 0.5) (layer F.Cu) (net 14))
 (segment (start 146.58 134.58) (end 149.5 137.5) (width 0.5) (layer F.Cu) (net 14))
 (segment (start 149.5 137.5) (end 152.73 137.5) (width 0.5) (layer F.Cu) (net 14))
 (segment (start 163.38 109.1) (end 165.6 109.7) (width 0.5) (layer F.Cu) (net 15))
 (segment (start 165.6 109.7) (end 166.33 108.97) (width 0.5) (layer F.Cu) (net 15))
 (segment (start 166.33 108.97) (end 168.3 108.97) (width 0.5) (layer F.Cu) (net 15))
 (segment (start 125.92 101) (end 125.92 105) (width 0.5) (layer F.Cu) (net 18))
 (segment (start 131 126.5) (end 131 129.42) (width 0.5) (layer F.Cu) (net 16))
 (segment (start 131 129.42) (end 133.08 131.5) (width 0.5) (layer F.Cu) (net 16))
 (segment (start 133.08 131.5) (end 136.42 131.5) (width 0.5) (layer F.Cu) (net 16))
 (segment (start 140.69 119.08) (end 140.69 121.62) (width 0.5) (layer F.Cu) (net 17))
 (segment (start 140.69 121.62) (end 138.42 121.62) (width 0.5) (layer F.Cu) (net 17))
 (segment (start 138.42 121.62) (end 133.54 126.5) (width 0.5) (layer F.Cu) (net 17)))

